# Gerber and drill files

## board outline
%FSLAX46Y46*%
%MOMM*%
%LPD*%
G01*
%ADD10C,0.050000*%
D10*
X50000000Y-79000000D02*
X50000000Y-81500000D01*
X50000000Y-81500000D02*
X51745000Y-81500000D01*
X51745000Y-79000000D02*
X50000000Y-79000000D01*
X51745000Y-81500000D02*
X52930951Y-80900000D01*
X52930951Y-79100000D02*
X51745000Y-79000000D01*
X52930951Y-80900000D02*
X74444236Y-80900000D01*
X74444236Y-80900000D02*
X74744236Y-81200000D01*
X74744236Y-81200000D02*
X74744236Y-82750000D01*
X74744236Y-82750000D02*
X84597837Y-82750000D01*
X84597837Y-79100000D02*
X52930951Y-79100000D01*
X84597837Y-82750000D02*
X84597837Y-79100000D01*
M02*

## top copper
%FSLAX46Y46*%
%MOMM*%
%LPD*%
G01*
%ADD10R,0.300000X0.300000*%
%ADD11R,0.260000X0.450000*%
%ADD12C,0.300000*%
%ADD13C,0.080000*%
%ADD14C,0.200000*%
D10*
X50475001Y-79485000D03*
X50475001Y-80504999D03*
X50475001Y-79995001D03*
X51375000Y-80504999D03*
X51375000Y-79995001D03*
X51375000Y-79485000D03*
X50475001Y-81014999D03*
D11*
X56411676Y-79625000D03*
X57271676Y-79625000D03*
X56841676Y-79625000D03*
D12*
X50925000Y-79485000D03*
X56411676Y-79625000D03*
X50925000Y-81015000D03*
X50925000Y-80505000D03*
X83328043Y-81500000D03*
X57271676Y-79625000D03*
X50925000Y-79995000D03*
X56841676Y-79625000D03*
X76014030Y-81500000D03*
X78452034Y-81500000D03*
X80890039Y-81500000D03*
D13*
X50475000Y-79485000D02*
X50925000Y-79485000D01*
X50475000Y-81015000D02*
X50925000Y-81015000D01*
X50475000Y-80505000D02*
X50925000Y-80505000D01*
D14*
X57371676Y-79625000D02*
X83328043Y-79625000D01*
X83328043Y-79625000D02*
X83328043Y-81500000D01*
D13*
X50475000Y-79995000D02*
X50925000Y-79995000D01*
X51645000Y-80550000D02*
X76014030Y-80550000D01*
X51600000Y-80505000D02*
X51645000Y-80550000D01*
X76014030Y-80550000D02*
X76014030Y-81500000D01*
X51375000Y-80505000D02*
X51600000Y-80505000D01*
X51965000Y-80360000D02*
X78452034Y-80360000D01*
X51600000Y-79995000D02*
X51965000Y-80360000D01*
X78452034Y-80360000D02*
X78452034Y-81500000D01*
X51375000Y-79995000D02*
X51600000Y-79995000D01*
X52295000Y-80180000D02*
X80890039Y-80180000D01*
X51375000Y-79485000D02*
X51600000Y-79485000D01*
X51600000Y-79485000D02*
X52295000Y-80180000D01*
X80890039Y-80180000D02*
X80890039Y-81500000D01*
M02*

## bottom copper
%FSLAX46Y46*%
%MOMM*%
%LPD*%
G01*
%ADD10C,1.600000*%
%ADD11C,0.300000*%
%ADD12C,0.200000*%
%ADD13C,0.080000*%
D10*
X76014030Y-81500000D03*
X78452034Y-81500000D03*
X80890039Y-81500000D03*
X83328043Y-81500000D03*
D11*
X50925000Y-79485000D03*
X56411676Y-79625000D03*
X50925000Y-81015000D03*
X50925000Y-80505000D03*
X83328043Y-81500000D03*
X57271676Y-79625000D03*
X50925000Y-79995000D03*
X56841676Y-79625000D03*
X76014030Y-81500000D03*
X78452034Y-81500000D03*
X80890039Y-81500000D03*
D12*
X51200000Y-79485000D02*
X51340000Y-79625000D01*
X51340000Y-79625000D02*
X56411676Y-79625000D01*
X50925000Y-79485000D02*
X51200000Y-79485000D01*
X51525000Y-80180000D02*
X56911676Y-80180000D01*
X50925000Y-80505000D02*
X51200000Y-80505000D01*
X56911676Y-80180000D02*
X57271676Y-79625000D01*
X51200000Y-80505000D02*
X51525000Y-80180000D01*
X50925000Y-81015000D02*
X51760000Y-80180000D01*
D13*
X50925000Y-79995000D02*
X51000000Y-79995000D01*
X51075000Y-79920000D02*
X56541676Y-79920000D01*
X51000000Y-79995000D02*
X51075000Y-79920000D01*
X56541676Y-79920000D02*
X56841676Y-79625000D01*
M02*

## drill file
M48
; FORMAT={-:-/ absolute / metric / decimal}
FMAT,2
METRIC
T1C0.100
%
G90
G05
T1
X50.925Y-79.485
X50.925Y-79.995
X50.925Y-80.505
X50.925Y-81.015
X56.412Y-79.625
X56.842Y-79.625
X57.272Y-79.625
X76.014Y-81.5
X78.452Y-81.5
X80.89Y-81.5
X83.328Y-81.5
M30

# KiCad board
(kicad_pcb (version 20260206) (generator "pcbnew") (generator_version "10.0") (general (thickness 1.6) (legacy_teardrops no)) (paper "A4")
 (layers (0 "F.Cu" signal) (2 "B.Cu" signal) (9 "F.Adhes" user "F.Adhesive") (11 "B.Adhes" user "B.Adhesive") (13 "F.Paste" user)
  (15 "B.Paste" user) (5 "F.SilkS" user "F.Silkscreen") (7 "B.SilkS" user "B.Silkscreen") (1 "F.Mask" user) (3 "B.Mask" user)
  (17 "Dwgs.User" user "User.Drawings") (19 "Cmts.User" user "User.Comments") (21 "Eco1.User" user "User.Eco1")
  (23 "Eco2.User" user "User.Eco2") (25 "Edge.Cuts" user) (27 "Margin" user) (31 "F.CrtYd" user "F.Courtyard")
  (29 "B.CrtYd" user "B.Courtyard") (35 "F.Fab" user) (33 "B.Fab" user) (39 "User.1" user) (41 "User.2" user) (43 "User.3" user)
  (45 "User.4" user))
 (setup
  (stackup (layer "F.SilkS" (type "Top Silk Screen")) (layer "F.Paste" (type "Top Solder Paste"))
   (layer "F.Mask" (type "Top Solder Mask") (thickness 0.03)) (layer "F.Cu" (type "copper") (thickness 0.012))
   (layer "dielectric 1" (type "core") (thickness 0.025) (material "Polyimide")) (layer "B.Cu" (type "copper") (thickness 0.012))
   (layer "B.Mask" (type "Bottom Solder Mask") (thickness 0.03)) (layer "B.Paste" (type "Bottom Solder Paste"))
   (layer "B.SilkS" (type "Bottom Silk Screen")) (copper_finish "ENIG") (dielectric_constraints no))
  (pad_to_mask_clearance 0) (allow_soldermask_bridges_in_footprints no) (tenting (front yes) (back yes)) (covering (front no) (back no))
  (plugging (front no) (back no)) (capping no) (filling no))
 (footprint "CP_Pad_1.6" (layer "F.Cu") (at 76.01403 81.5)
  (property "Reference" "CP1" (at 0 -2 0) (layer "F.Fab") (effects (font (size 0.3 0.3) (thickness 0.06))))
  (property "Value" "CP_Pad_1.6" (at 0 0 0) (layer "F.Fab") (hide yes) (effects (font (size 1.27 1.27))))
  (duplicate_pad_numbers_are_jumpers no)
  (pad "1" smd circle (at 0 0) (size 1.6 1.6) (layers "B.Cu" "B.Mask") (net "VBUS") (solder_mask_margin 0.1)))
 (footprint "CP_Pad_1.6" (layer "F.Cu") (at 83.328043 81.5)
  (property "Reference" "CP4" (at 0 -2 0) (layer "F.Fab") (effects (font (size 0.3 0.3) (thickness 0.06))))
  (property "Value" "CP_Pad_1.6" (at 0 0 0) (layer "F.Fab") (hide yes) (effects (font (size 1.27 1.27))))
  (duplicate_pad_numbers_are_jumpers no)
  (pad "1" smd circle (at 0 0) (size 1.6 1.6) (layers "B.Cu" "B.Mask") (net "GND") (solder_mask_margin 0.1)))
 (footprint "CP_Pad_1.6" (layer "F.Cu") (at 80.890039 81.5)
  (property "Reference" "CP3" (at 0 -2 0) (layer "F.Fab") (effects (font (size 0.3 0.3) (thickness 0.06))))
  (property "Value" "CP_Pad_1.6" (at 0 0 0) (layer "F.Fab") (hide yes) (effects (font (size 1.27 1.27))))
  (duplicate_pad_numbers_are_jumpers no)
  (pad "1" smd circle (at 0 0) (size 1.6 1.6) (layers "B.Cu" "B.Mask") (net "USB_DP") (solder_mask_margin 0.1)))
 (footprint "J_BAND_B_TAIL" (layer "F.Cu") (at 50.9 80.25)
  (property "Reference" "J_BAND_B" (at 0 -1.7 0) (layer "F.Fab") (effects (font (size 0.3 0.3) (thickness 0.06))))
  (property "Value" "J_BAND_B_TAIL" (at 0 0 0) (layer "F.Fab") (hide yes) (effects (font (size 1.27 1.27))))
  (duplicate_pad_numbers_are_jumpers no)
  (pad "1" smd rect (at -0.424999 -0.765) (size 0.3 0.3) (layers "F.Cu" "F.Mask") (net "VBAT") (solder_mask_margin 0.05)
   (thermal_bridge_angle 45))
  (pad "2" smd rect (at -0.424999 0.254999) (size 0.3 0.3) (layers "F.Cu" "F.Mask") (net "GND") (solder_mask_margin 0.05)
   (thermal_bridge_angle 45))
  (pad "3" smd rect (at -0.424999 -0.254999) (size 0.3 0.3) (layers "F.Cu" "F.Mask") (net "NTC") (solder_mask_margin 0.05)
   (thermal_bridge_angle 45))
  (pad "4" smd rect (at 0.475 0.254999) (size 0.3 0.3) (layers "F.Cu" "F.Mask") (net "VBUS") (solder_mask_margin 0.05)
   (thermal_bridge_angle 45))
  (pad "5" smd rect (at 0.475 -0.254999) (size 0.3 0.3) (layers "F.Cu" "F.Mask") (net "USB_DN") (solder_mask_margin 0.05)
   (thermal_bridge_angle 45))
  (pad "6" smd rect (at 0.475 -0.765) (size 0.3 0.3) (layers "F.Cu" "F.Mask") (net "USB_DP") (solder_mask_margin 0.05)
   (thermal_bridge_angle 45))
  (pad "7" smd rect (at -0.424999 0.764999) (size 0.3 0.3) (layers "F.Cu" "F.Mask") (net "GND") (solder_mask_margin 0.05)
   (thermal_bridge_angle 45)))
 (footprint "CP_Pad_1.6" (layer "F.Cu") (at 78.452034 81.5)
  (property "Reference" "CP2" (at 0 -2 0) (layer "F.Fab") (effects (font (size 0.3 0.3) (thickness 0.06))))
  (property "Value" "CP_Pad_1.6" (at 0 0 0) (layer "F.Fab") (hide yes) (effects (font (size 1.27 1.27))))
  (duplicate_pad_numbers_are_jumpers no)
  (pad "1" smd circle (at 0 0) (size 1.6 1.6) (layers "B.Cu" "B.Mask") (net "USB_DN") (solder_mask_margin 0.1)))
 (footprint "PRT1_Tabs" (layer "F.Cu") (at 56.841676 79.625)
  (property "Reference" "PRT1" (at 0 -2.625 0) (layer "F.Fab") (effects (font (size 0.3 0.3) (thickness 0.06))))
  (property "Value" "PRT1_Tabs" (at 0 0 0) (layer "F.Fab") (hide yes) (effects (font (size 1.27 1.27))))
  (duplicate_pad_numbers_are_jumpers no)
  (pad "1" smd rect (at -0.43 0) (size 0.26 0.45) (layers "F.Cu" "F.Mask") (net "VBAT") (solder_mask_margin 0.05) (thermal_bridge_angle 45))
  (pad "2" smd rect (at 0.43 0) (size 0.26 0.45) (layers "F.Cu" "F.Mask") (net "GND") (solder_mask_margin 0.05) (thermal_bridge_angle 45))
  (pad "3" smd rect (at 0 0) (size 0.26 0.45) (layers "F.Cu" "F.Mask") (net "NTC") (solder_mask_margin 0.05) (thermal_bridge_angle 45)))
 (gr_line (start 50 79) (end 50 81.5) (stroke (width 0.05) (type default)) (layer "Edge.Cuts"))
 (gr_line (start 50 81.5) (end 51.745 81.5) (stroke (width 0.05) (type default)) (layer "Edge.Cuts"))
 (gr_line (start 51.745 79) (end 50 79) (stroke (width 0.05) (type default)) (layer "Edge.Cuts"))
 (gr_line (start 51.745 81.5) (end 52.930951 80.9) (stroke (width 0.05) (type default)) (layer "Edge.Cuts"))
 (gr_line (start 52.930951 79.1) (end 51.745 79) (stroke (width 0.05) (type default)) (layer "Edge.Cuts"))
 (gr_line (start 52.930951 80.9) (end 74.444236 80.9) (stroke (width 0.05) (type default)) (layer "Edge.Cuts"))
 (gr_line (start 74.444236 80.9) (end 74.744236 81.2) (stroke (width 0.05) (type default)) (layer "Edge.Cuts"))
 (gr_line (start 74.744236 81.2) (end 74.744236 82.75) (stroke (width 0.05) (type default)) (layer "Edge.Cuts"))
 (gr_line (start 74.744236 82.75) (end 84.597837 82.75) (stroke (width 0.05) (type default)) (layer "Edge.Cuts"))
 (gr_line (start 84.597837 79.1) (end 52.930951 79.1) (stroke (width 0.05) (type default)) (layer "Edge.Cuts"))
 (gr_line (start 84.597837 82.75) (end 84.597837 79.1) (stroke (width 0.05) (type default)) (layer "Edge.Cuts"))
 (segment (start 50.475 79.485) (end 50.925 79.485) (width 0.08) (layer "F.Cu") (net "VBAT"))
 (via (at 50.925 79.485) (size 0.3) (drill 0.1) (layers "F.Cu" "B.Cu") (tenting (front yes) (back yes)) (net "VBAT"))
 (via (at 56.411676 79.625) (size 0.3) (drill 0.1) (layers "F.Cu" "B.Cu") (tenting (front yes) (back yes)) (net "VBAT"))
 (segment (start 50.925 79.485) (end 51.2 79.485) (width 0.2) (layer "B.Cu") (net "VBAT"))
 (segment (start 51.34 79.625) (end 56.411676 79.625) (width 0.2) (layer "B.Cu") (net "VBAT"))
 (segment (start 51.2 79.485) (end 51.34 79.625) (width 0.2) (layer "B.Cu") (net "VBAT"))
 (segment (start 57.371676 79.625) (end 83.328043 79.625) (width 0.2) (layer "F.Cu") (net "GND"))
 (segment (start 50.475 81.015) (end 50.925 81.015) (width 0.08) (layer "F.Cu") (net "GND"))
 (segment (start 50.475 80.505) (end 50.925 80.505) (width 0.08) (layer "F.Cu") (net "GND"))
 (segment (start 83.328043 79.625) (end 83.328043 81.5) (width 0.2) (layer "F.Cu") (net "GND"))
 (via (at 57.271676 79.625) (size 0.3) (drill 0.1) (layers "F.Cu" "B.Cu") (tenting (front yes) (back yes)) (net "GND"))
 (via (at 50.925 80.505) (size 0.3) (drill 0.1) (layers "F.Cu" "B.Cu") (tenting (front yes) (back yes)) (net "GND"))
 (via (at 50.925 81.015) (size 0.3) (drill 0.1) (layers "F.Cu" "B.Cu") (tenting (front yes) (back yes)) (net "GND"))
 (via (at 83.328043 81.5) (size 0.3) (drill 0.1) (layers "F.Cu" "B.Cu") (tenting (front yes) (back yes)) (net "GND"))
 (segment (start 50.925 80.505) (end 51.2 80.505) (width 0.2) (layer "B.Cu") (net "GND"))
 (segment (start 51.525 80.18) (end 56.911676 80.18) (width 0.2) (layer "B.Cu") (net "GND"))
 (segment (start 51.2 80.505) (end 51.525 80.18) (width 0.2) (layer "B.Cu") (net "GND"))
 (segment (start 56.911676 80.18) (end 57.271676 79.625) (width 0.2) (layer "B.Cu") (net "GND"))
 (segment (start 50.925 81.015) (end 51.76 80.18) (width 0.2) (layer "B.Cu") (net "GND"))
 (segment (start 50.475 79.995) (end 50.925 79.995) (width 0.08) (layer "F.Cu") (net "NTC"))
 (via (at 50.925 79.995) (size 0.3) (drill 0.1) (layers "F.Cu" "B.Cu") (tenting (front yes) (back yes)) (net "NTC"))
 (via (at 56.841676 79.625) (size 0.3) (drill 0.1) (layers "F.Cu" "B.Cu") (tenting (front yes) (back yes)) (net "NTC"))
 (segment (start 51 79.995) (end 51.075 79.92) (width 0.08) (layer "B.Cu") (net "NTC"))
 (segment (start 56.541676 79.92) (end 56.841676 79.625) (width 0.08) (layer "B.Cu") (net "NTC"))
 (segment (start 51.075 79.92) (end 56.541676 79.92) (width 0.08) (layer "B.Cu") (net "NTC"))
 (segment (start 50.925 79.995) (end 51 79.995) (width 0.08) (layer "B.Cu") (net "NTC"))
 (segment (start 51.375 80.505) (end 51.6 80.505) (width 0.08) (layer "F.Cu") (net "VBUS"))
 (segment (start 51.645 80.55) (end 76.01403 80.55) (width 0.08) (layer "F.Cu") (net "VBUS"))
 (segment (start 76.01403 80.55) (end 76.01403 81.5) (width 0.08) (layer "F.Cu") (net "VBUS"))
 (segment (start 51.6 80.505) (end 51.645 80.55) (width 0.08) (layer "F.Cu") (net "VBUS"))
 (via (at 76.01403 81.5) (size 0.3) (drill 0.1) (layers "F.Cu" "B.Cu") (tenting (front yes) (back yes)) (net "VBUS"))
 (segment (start 51.375 79.995) (end 51.6 79.995) (width 0.08) (layer "F.Cu") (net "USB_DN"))
 (segment (start 51.6 79.995) (end 51.965 80.36) (width 0.08) (layer "F.Cu") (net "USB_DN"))
 (segment (start 51.965 80.36) (end 78.452034 80.36) (width 0.08) (layer "F.Cu") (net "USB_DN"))
 (segment (start 78.452034 80.36) (end 78.452034 81.5) (width 0.08) (layer "F.Cu") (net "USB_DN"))
 (via (at 78.452034 81.5) (size 0.3) (drill 0.1) (layers "F.Cu" "B.Cu") (tenting (front yes) (back yes)) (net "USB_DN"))
 (segment (start 52.295 80.18) (end 80.890039 80.18) (width 0.08) (layer "F.Cu") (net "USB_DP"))
 (segment (start 51.6 79.485) (end 52.295 80.18) (width 0.08) (layer "F.Cu") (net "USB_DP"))
 (segment (start 80.890039 80.18) (end 80.890039 81.5) (width 0.08) (layer "F.Cu") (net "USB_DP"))
 (segment (start 51.375 79.485) (end 51.6 79.485) (width 0.08) (layer "F.Cu") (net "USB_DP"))
 (via (at 80.890039 81.5) (size 0.3) (drill 0.1) (layers "F.Cu" "B.Cu") (tenting (front yes) (back yes)) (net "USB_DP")))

